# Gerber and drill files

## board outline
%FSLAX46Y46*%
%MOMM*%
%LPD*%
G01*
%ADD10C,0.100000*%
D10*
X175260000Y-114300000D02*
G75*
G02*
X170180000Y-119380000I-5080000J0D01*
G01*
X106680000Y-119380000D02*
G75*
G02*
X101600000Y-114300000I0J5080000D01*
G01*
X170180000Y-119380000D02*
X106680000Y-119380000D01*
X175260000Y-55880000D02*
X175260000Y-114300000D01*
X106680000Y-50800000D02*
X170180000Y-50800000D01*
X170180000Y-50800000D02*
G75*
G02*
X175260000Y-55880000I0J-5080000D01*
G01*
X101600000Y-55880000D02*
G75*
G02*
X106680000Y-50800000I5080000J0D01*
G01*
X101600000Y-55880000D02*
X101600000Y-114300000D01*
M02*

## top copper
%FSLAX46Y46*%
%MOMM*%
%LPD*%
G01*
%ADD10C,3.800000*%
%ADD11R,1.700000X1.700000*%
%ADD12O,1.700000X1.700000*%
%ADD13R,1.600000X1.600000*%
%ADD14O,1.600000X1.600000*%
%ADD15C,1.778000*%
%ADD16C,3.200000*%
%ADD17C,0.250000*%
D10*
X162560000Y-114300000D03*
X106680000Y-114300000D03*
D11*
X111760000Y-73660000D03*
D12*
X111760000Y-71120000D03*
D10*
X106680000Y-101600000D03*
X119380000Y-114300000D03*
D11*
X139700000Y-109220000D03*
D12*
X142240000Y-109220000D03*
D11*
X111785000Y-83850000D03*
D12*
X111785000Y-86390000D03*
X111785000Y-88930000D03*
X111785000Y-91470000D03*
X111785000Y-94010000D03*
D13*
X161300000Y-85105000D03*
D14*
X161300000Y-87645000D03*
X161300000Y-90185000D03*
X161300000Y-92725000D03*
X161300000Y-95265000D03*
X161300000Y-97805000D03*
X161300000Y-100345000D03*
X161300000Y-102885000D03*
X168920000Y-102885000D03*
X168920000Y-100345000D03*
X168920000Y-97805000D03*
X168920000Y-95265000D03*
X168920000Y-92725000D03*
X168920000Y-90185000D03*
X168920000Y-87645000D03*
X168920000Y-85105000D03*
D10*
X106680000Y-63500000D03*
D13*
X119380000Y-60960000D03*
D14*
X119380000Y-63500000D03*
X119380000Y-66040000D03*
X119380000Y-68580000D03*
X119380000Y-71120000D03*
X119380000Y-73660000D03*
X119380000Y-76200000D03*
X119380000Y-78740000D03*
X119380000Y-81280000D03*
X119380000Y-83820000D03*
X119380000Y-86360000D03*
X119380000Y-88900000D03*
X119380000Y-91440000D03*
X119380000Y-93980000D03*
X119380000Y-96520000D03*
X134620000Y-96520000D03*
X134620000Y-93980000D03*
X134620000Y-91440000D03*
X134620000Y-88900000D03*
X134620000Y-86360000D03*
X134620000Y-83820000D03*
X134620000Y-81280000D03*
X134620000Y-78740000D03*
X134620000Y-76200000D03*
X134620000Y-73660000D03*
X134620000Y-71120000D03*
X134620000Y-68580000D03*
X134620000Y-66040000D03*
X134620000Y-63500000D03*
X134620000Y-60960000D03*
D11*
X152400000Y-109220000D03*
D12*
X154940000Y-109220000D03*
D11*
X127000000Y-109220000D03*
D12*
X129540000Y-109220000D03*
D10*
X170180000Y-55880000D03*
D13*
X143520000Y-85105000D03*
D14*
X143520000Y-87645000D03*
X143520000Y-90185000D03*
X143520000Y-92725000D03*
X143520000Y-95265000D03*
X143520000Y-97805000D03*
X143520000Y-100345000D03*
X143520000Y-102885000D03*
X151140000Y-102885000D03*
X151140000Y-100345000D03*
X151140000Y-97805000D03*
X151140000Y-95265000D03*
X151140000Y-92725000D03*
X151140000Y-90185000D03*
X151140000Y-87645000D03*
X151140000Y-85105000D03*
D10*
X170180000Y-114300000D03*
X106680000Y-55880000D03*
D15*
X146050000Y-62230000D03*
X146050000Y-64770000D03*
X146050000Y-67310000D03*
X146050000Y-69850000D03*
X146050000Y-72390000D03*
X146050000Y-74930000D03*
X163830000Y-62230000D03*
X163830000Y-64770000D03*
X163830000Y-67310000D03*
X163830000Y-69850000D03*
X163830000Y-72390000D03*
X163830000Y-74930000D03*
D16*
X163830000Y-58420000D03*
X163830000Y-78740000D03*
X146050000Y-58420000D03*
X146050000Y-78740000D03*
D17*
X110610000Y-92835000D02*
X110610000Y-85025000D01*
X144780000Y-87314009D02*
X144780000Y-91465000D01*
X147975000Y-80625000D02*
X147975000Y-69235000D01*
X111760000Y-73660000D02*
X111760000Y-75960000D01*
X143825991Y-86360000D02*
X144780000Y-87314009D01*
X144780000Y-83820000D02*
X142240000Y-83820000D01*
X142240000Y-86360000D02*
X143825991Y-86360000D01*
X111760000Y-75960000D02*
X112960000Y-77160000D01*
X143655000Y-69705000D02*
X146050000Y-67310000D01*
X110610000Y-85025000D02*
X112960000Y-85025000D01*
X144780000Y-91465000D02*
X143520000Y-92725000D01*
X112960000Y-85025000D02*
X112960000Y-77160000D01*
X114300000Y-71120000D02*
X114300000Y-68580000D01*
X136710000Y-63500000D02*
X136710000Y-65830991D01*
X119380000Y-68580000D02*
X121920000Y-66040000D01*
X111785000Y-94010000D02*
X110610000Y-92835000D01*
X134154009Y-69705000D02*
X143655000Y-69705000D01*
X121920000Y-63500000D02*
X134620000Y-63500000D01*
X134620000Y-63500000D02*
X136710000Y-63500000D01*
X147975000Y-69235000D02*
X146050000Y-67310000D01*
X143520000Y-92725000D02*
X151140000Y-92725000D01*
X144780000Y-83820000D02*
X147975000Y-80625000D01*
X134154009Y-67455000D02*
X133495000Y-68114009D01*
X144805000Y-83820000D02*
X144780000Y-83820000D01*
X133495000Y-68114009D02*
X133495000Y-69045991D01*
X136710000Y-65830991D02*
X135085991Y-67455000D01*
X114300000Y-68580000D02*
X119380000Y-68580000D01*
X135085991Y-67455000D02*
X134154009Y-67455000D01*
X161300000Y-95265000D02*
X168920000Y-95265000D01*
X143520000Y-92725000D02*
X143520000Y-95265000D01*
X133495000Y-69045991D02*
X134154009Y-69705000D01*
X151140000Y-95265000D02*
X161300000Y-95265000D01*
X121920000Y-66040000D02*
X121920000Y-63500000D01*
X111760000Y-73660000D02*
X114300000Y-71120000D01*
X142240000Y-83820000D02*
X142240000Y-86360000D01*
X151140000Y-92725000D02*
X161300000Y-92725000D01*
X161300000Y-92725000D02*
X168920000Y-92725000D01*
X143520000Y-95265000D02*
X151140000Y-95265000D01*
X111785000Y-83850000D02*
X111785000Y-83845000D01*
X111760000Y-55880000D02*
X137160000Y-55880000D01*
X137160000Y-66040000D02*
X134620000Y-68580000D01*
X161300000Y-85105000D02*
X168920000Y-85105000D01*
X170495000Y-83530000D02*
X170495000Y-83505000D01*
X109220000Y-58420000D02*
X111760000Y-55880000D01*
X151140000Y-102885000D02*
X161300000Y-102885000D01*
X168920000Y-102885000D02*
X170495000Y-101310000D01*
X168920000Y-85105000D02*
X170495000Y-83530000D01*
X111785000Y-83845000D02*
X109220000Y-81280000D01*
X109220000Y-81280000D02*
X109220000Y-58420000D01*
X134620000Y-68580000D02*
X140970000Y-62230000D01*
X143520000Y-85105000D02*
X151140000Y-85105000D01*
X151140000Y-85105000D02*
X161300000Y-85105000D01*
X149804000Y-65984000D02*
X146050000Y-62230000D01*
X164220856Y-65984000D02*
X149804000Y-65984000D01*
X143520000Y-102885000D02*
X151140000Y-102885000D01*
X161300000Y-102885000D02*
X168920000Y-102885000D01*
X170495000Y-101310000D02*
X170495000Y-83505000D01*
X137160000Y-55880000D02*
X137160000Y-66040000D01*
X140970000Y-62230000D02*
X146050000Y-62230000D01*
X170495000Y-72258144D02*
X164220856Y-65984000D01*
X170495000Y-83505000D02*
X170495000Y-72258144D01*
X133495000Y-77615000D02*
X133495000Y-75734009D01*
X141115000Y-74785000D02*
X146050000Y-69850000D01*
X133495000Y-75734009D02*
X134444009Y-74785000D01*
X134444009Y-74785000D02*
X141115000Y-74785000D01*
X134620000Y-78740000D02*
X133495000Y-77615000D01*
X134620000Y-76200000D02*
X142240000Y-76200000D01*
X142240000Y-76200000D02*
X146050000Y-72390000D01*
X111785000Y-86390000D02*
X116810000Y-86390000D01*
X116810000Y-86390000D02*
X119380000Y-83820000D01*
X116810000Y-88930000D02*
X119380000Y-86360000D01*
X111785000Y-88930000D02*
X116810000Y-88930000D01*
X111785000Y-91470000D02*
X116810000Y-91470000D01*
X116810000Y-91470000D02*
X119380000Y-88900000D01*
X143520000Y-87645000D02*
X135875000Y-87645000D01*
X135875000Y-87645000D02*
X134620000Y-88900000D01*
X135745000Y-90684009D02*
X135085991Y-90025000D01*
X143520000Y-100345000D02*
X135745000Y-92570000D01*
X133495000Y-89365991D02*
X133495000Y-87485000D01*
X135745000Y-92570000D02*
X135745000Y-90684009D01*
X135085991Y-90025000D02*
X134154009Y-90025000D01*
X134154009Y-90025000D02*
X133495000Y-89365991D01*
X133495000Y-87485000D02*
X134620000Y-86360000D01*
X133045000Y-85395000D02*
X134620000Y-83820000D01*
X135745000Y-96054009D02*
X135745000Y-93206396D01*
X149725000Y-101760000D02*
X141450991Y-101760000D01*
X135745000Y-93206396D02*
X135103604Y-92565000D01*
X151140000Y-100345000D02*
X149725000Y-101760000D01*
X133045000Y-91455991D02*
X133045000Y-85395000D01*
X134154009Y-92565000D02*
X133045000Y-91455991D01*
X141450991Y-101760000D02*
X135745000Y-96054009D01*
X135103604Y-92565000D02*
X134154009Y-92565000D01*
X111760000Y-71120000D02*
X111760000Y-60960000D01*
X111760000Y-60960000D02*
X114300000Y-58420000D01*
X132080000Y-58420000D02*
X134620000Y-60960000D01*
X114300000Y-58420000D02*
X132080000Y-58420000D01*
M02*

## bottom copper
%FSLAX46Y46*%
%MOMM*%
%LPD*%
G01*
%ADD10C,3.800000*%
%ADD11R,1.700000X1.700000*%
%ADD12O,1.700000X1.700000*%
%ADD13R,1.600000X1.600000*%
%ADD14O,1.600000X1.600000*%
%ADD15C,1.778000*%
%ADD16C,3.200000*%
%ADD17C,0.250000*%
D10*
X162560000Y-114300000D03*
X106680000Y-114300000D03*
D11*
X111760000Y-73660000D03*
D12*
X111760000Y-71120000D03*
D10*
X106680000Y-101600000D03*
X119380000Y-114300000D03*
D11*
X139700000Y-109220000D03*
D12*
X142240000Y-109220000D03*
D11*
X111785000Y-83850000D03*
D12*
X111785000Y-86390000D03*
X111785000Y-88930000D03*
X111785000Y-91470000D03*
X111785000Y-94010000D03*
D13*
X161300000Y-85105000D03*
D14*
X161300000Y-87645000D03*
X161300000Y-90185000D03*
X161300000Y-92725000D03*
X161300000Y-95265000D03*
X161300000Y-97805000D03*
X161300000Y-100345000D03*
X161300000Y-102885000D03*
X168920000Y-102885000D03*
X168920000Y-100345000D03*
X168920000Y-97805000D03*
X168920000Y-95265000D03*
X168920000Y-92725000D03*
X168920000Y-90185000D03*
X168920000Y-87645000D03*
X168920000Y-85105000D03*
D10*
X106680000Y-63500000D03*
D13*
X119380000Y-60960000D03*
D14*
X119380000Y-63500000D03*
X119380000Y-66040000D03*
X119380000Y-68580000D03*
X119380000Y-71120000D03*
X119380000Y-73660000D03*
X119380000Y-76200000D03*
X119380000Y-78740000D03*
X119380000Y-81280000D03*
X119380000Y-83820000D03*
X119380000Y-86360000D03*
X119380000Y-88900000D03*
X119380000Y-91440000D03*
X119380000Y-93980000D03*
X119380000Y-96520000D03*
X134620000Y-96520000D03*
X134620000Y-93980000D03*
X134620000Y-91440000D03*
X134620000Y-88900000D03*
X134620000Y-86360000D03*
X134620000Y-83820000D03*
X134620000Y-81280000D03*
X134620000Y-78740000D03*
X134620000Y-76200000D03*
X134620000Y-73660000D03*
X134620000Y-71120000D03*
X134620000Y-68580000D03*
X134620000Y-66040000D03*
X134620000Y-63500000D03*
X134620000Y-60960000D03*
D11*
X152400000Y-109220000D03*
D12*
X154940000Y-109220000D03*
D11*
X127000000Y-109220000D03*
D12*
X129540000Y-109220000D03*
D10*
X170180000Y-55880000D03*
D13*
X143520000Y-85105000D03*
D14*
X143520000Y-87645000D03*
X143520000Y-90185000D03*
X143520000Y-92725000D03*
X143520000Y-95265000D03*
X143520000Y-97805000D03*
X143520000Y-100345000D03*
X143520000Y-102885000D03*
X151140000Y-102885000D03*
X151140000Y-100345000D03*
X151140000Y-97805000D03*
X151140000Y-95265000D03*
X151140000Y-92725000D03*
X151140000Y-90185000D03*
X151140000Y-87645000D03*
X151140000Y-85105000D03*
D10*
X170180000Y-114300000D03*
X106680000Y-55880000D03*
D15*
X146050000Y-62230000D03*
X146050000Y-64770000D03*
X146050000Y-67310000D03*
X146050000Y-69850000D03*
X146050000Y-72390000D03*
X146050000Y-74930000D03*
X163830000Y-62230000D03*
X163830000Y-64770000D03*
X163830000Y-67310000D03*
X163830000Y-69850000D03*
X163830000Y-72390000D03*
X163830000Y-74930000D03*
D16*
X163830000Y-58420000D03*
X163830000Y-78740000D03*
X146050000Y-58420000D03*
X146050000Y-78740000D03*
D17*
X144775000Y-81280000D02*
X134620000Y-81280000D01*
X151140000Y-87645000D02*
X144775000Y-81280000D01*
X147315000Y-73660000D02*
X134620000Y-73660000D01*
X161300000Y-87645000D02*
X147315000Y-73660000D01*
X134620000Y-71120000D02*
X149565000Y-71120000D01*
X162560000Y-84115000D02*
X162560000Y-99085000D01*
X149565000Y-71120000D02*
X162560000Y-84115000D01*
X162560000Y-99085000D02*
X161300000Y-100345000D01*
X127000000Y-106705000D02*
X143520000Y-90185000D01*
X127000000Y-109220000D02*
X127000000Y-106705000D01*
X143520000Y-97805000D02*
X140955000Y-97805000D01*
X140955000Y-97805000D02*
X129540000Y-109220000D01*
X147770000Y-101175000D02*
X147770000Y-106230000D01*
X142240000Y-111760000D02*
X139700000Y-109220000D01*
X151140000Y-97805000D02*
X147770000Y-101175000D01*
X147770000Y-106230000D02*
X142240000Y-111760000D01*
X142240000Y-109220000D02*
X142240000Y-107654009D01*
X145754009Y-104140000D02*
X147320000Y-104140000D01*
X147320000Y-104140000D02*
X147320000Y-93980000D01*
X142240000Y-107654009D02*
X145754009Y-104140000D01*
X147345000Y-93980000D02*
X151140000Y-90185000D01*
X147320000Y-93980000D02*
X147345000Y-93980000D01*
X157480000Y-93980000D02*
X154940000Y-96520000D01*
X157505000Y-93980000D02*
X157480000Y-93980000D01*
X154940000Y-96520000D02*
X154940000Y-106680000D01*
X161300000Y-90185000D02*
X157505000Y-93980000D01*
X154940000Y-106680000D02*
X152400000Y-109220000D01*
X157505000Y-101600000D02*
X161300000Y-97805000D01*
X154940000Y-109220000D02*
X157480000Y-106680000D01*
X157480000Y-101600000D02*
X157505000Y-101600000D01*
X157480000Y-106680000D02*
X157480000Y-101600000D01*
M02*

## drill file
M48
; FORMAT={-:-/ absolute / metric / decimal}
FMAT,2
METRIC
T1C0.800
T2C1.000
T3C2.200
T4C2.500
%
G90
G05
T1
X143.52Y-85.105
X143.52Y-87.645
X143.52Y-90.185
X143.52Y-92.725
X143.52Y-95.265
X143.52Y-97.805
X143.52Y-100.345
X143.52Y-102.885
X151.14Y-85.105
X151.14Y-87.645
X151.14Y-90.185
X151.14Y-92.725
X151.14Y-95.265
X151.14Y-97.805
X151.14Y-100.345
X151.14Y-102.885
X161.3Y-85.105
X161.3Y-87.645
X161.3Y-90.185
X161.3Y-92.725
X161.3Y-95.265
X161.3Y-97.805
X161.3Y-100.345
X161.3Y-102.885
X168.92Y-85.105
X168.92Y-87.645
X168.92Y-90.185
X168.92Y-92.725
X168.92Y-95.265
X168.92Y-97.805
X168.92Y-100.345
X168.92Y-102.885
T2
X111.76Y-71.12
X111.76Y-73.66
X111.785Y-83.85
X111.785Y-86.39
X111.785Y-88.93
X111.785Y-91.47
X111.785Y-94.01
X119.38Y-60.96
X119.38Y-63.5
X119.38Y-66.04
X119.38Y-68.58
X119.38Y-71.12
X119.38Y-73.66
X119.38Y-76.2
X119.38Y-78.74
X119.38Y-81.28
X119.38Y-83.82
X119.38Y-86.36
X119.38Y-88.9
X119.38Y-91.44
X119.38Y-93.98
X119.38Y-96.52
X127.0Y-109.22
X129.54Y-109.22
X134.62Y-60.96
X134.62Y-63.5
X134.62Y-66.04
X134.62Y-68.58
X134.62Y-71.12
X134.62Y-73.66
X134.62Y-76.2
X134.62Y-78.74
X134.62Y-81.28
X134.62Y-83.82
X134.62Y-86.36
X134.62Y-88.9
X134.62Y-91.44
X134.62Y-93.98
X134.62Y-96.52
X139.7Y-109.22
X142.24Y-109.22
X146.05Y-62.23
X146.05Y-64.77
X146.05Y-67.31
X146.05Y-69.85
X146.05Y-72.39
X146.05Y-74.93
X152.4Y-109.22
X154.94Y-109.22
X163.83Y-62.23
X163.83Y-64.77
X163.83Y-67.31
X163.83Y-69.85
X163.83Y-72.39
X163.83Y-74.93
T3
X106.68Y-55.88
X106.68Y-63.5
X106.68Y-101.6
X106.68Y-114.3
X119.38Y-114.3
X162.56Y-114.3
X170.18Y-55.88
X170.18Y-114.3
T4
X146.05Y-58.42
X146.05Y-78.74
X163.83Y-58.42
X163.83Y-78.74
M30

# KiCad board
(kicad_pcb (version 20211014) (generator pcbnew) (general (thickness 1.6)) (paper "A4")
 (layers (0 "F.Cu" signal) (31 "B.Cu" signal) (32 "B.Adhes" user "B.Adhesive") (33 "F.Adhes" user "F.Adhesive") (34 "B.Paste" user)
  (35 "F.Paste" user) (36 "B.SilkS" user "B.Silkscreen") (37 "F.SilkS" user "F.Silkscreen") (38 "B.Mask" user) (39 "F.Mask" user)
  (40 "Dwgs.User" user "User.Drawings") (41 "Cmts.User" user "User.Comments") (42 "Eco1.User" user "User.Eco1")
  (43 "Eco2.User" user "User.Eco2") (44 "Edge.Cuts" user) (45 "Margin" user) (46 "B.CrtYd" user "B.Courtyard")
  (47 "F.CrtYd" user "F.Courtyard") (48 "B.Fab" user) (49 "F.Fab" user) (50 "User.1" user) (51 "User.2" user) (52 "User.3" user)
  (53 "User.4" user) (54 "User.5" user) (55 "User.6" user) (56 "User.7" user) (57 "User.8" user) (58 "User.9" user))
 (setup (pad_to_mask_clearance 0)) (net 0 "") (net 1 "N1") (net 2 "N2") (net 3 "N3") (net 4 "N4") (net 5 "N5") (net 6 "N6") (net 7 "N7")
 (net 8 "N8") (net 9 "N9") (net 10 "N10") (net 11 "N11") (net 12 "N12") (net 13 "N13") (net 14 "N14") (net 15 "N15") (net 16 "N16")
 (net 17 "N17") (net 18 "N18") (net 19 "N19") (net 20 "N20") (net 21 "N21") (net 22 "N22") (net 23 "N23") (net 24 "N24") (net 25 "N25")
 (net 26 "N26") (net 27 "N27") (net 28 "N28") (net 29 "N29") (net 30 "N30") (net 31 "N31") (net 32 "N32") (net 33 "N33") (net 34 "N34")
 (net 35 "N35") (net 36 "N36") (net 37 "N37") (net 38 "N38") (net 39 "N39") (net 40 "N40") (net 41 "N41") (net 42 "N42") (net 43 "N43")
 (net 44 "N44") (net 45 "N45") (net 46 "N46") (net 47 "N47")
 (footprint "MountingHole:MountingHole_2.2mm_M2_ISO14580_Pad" (layer "F.Cu") (at 162.56 114.3)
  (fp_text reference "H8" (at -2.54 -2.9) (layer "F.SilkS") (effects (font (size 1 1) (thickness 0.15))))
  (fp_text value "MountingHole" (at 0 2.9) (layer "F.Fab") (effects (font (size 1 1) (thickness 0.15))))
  (pad "1" thru_hole circle (at 0 0) (size 3.8 3.8) (drill 2.2) (layers *.Cu *.Mask)))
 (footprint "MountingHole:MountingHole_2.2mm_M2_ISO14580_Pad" (layer "F.Cu") (at 106.68 114.3)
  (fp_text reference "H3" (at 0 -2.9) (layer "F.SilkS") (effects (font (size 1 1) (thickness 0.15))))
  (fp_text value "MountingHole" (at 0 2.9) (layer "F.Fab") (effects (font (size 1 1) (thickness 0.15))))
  (pad "1" thru_hole circle (at 0 0) (size 3.8 3.8) (drill 2.2) (layers *.Cu *.Mask)))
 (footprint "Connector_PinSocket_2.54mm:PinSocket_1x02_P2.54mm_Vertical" (layer "F.Cu") (at 111.76 73.66 180)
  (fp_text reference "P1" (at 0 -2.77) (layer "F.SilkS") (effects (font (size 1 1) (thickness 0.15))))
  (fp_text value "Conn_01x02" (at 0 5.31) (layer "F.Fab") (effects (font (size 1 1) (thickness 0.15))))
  (pad "1" thru_hole rect (at 0 0 180) (size 1.7 1.7) (drill 1) (layers *.Cu *.Mask) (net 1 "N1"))
  (pad "2" thru_hole oval (at 0 2.54 180) (size 1.7 1.7) (drill 1) (layers *.Cu *.Mask) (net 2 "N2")))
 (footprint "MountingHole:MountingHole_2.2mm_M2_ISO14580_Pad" (layer "F.Cu") (at 106.68 101.6)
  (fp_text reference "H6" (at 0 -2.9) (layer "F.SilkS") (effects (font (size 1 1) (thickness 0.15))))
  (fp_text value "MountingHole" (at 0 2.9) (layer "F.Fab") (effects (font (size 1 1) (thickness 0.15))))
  (pad "1" thru_hole circle (at 0 0) (size 3.8 3.8) (drill 2.2) (layers *.Cu *.Mask)))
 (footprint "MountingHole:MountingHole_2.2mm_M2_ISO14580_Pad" (layer "F.Cu") (at 119.38 114.3)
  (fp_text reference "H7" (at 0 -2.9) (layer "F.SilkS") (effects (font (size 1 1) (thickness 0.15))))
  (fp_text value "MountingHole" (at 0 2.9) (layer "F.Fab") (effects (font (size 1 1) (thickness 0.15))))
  (pad "1" thru_hole circle (at 0 0) (size 3.8 3.8) (drill 2.2) (layers *.Cu *.Mask)))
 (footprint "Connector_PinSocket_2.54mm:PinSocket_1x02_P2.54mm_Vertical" (layer "F.Cu") (at 139.7 109.22 90)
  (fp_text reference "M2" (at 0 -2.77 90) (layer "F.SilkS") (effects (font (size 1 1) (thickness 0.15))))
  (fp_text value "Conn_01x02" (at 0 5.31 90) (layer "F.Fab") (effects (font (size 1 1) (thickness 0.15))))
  (pad "1" thru_hole rect (at 0 0 90) (size 1.7 1.7) (drill 1) (layers *.Cu *.Mask) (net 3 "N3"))
  (pad "2" thru_hole oval (at 0 2.54 90) (size 1.7 1.7) (drill 1) (layers *.Cu *.Mask) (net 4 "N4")))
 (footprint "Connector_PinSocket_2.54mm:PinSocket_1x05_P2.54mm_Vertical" (layer "F.Cu") (at 111.785 83.85)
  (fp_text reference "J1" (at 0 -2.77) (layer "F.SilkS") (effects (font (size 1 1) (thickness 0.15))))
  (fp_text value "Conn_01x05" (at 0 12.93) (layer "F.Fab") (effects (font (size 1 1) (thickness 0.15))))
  (pad "1" thru_hole rect (at 0 0) (size 1.7 1.7) (drill 1) (layers *.Cu *.Mask) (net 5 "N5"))
  (pad "2" thru_hole oval (at 0 2.54) (size 1.7 1.7) (drill 1) (layers *.Cu *.Mask) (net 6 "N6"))
  (pad "3" thru_hole oval (at 0 5.08) (size 1.7 1.7) (drill 1) (layers *.Cu *.Mask) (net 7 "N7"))
  (pad "4" thru_hole oval (at 0 7.62) (size 1.7 1.7) (drill 1) (layers *.Cu *.Mask) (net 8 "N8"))
  (pad "5" thru_hole oval (at 0 10.16) (size 1.7 1.7) (drill 1) (layers *.Cu *.Mask) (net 1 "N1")))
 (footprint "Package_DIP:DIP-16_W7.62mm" (layer "F.Cu") (at 161.3 85.105)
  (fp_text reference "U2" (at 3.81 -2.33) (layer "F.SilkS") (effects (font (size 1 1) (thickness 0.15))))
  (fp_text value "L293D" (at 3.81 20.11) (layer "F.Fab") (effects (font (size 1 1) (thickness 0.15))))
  (pad "1" thru_hole rect (at 0 0) (size 1.6 1.6) (drill 0.8) (layers *.Cu *.Mask) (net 5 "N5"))
  (pad "2" thru_hole oval (at 0 2.54) (size 1.6 1.6) (drill 0.8) (layers *.Cu *.Mask) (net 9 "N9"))
  (pad "3" thru_hole oval (at 0 5.08) (size 1.6 1.6) (drill 0.8) (layers *.Cu *.Mask) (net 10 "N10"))
  (pad "4" thru_hole oval (at 0 7.62) (size 1.6 1.6) (drill 0.8) (layers *.Cu *.Mask) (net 1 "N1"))
  (pad "5" thru_hole oval (at 0 10.16) (size 1.6 1.6) (drill 0.8) (layers *.Cu *.Mask) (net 1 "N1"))
  (pad "6" thru_hole oval (at 0 12.7) (size 1.6 1.6) (drill 0.8) (layers *.Cu *.Mask) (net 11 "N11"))
  (pad "7" thru_hole oval (at 0 15.24) (size 1.6 1.6) (drill 0.8) (layers *.Cu *.Mask) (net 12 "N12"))
  (pad "8" thru_hole oval (at 0 17.78) (size 1.6 1.6) (drill 0.8) (layers *.Cu *.Mask) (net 5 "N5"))
  (pad "9" thru_hole oval (at 7.62 17.78) (size 1.6 1.6) (drill 0.8) (layers *.Cu *.Mask) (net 5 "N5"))
  (pad "10" thru_hole oval (at 7.62 15.24) (size 1.6 1.6) (drill 0.8) (layers *.Cu *.Mask) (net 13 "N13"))
  (pad "11" thru_hole oval (at 7.62 12.7) (size 1.6 1.6) (drill 0.8) (layers *.Cu *.Mask) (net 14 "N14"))
  (pad "12" thru_hole oval (at 7.62 10.16) (size 1.6 1.6) (drill 0.8) (layers *.Cu *.Mask) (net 1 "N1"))
  (pad "13" thru_hole oval (at 7.62 7.62) (size 1.6 1.6) (drill 0.8) (layers *.Cu *.Mask) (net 1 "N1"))
  (pad "14" thru_hole oval (at 7.62 5.08) (size 1.6 1.6) (drill 0.8) (layers *.Cu *.Mask) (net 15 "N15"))
  (pad "15" thru_hole oval (at 7.62 2.54) (size 1.6 1.6) (drill 0.8) (layers *.Cu *.Mask) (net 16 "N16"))
  (pad "16" thru_hole oval (at 7.62 0) (size 1.6 1.6) (drill 0.8) (layers *.Cu *.Mask) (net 5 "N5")))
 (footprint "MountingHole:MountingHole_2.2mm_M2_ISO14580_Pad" (layer "F.Cu") (at 106.68 63.5)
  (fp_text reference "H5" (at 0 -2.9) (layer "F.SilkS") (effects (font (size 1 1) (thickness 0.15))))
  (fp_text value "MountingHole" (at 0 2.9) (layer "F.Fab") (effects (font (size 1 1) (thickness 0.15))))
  (pad "1" thru_hole circle (at 0 0) (size 3.8 3.8) (drill 2.2) (layers *.Cu *.Mask)))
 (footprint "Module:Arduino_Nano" (layer "F.Cu") (at 119.38 60.96)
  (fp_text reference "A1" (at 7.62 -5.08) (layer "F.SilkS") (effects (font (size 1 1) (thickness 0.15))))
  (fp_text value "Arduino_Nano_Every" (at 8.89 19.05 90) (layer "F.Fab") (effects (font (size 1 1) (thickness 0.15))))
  (pad "1" thru_hole rect (at 0 0) (size 1.6 1.6) (drill 1) (layers *.Cu *.Mask) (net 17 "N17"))
  (pad "2" thru_hole oval (at 0 2.54) (size 1.6 1.6) (drill 1) (layers *.Cu *.Mask) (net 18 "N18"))
  (pad "3" thru_hole oval (at 0 5.08) (size 1.6 1.6) (drill 1) (layers *.Cu *.Mask) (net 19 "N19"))
  (pad "4" thru_hole oval (at 0 7.62) (size 1.6 1.6) (drill 1) (layers *.Cu *.Mask) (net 1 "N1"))
  (pad "5" thru_hole oval (at 0 10.16) (size 1.6 1.6) (drill 1) (layers *.Cu *.Mask) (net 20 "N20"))
  (pad "6" thru_hole oval (at 0 12.7) (size 1.6 1.6) (drill 1) (layers *.Cu *.Mask) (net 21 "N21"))
  (pad "7" thru_hole oval (at 0 15.24) (size 1.6 1.6) (drill 1) (layers *.Cu *.Mask) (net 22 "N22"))
  (pad "8" thru_hole oval (at 0 17.78) (size 1.6 1.6) (drill 1) (layers *.Cu *.Mask) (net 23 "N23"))
  (pad "9" thru_hole oval (at 0 20.32) (size 1.6 1.6) (drill 1) (layers *.Cu *.Mask) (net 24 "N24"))
  (pad "10" thru_hole oval (at 0 22.86) (size 1.6 1.6) (drill 1) (layers *.Cu *.Mask) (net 6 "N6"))
  (pad "11" thru_hole oval (at 0 25.4) (size 1.6 1.6) (drill 1) (layers *.Cu *.Mask) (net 7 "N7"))
  (pad "12" thru_hole oval (at 0 27.94) (size 1.6 1.6) (drill 1) (layers *.Cu *.Mask) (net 8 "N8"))
  (pad "13" thru_hole oval (at 0 30.48) (size 1.6 1.6) (drill 1) (layers *.Cu *.Mask) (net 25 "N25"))
  (pad "14" thru_hole oval (at 0 33.02) (size 1.6 1.6) (drill 1) (layers *.Cu *.Mask) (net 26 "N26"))
  (pad "15" thru_hole oval (at 0 35.56) (size 1.6 1.6) (drill 1) (layers *.Cu *.Mask) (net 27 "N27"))
  (pad "16" thru_hole oval (at 15.24 35.56) (size 1.6 1.6) (drill 1) (layers *.Cu *.Mask) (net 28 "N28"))
  (pad "17" thru_hole oval (at 15.24 33.02) (size 1.6 1.6) (drill 1) (layers *.Cu *.Mask) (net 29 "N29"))
  (pad "18" thru_hole oval (at 15.24 30.48) (size 1.6 1.6) (drill 1) (layers *.Cu *.Mask) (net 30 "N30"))
  (pad "19" thru_hole oval (at 15.24 27.94) (size 1.6 1.6) (drill 1) (layers *.Cu *.Mask) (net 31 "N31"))
  (pad "20" thru_hole oval (at 15.24 25.4) (size 1.6 1.6) (drill 1) (layers *.Cu *.Mask) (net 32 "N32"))
  (pad "21" thru_hole oval (at 15.24 22.86) (size 1.6 1.6) (drill 1) (layers *.Cu *.Mask) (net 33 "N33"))
  (pad "22" thru_hole oval (at 15.24 20.32) (size 1.6 1.6) (drill 1) (layers *.Cu *.Mask) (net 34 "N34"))
  (pad "23" thru_hole oval (at 15.24 17.78) (size 1.6 1.6) (drill 1) (layers *.Cu *.Mask) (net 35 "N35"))
  (pad "24" thru_hole oval (at 15.24 15.24) (size 1.6 1.6) (drill 1) (layers *.Cu *.Mask) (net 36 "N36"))
  (pad "25" thru_hole oval (at 15.24 12.7) (size 1.6 1.6) (drill 1) (layers *.Cu *.Mask) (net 9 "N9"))
  (pad "26" thru_hole oval (at 15.24 10.16) (size 1.6 1.6) (drill 1) (layers *.Cu *.Mask) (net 12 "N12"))
  (pad "27" thru_hole oval (at 15.24 7.62) (size 1.6 1.6) (drill 1) (layers *.Cu *.Mask) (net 5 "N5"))
  (pad "28" thru_hole oval (at 15.24 5.08) (size 1.6 1.6) (drill 1) (layers *.Cu *.Mask) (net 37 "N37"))
  (pad "29" thru_hole oval (at 15.24 2.54) (size 1.6 1.6) (drill 1) (layers *.Cu *.Mask) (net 1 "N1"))
  (pad "30" thru_hole oval (at 15.24 0) (size 1.6 1.6) (drill 1) (layers *.Cu *.Mask) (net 2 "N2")))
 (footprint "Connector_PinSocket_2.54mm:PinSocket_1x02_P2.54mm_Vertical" (layer "F.Cu") (at 152.4 109.22 90)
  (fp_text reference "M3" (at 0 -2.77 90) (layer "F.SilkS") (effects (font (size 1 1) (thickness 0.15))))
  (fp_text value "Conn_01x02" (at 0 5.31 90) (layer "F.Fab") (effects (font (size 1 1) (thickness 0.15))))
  (pad "1" thru_hole rect (at 0 0 90) (size 1.7 1.7) (drill 1) (layers *.Cu *.Mask) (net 10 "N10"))
  (pad "2" thru_hole oval (at 0 2.54 90) (size 1.7 1.7) (drill 1) (layers *.Cu *.Mask) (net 11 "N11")))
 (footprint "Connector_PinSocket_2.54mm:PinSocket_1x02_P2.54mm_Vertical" (layer "F.Cu") (at 127 109.22 90)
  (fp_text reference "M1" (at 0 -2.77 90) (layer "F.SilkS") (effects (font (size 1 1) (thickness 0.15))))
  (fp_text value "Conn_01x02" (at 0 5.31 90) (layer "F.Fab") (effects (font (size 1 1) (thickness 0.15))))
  (pad "1" thru_hole rect (at 0 0 90) (size 1.7 1.7) (drill 1) (layers *.Cu *.Mask) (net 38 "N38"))
  (pad "2" thru_hole oval (at 0 2.54 90) (size 1.7 1.7) (drill 1) (layers *.Cu *.Mask) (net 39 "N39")))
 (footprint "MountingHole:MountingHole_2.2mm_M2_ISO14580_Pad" (layer "F.Cu") (at 170.18 55.88)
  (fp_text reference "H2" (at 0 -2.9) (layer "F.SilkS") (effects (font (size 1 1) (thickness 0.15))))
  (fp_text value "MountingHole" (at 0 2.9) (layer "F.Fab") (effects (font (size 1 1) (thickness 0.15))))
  (pad "1" thru_hole circle (at 0 0) (size 3.8 3.8) (drill 2.2) (layers *.Cu *.Mask)))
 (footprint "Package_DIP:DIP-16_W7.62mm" (layer "F.Cu") (at 143.52 85.105)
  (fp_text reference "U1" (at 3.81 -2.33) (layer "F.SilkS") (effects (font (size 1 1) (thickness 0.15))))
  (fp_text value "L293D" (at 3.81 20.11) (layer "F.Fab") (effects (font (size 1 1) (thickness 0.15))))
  (pad "1" thru_hole rect (at 0 0) (size 1.6 1.6) (drill 0.8) (layers *.Cu *.Mask) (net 5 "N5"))
  (pad "2" thru_hole oval (at 0 2.54) (size 1.6 1.6) (drill 0.8) (layers *.Cu *.Mask) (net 31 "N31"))
  (pad "3" thru_hole oval (at 0 5.08) (size 1.6 1.6) (drill 0.8) (layers *.Cu *.Mask) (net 38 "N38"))
  (pad "4" thru_hole oval (at 0 7.62) (size 1.6 1.6) (drill 0.8) (layers *.Cu *.Mask) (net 1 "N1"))
  (pad "5" thru_hole oval (at 0 10.16) (size 1.6 1.6) (drill 0.8) (layers *.Cu *.Mask) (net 1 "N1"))
  (pad "6" thru_hole oval (at 0 12.7) (size 1.6 1.6) (drill 0.8) (layers *.Cu *.Mask) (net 39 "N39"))
  (pad "7" thru_hole oval (at 0 15.24) (size 1.6 1.6) (drill 0.8) (layers *.Cu *.Mask) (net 32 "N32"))
  (pad "8" thru_hole oval (at 0 17.78) (size 1.6 1.6) (drill 0.8) (layers *.Cu *.Mask) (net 5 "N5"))
  (pad "9" thru_hole oval (at 7.62 17.78) (size 1.6 1.6) (drill 0.8) (layers *.Cu *.Mask) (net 5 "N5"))
  (pad "10" thru_hole oval (at 7.62 15.24) (size 1.6 1.6) (drill 0.8) (layers *.Cu *.Mask) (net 33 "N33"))
  (pad "11" thru_hole oval (at 7.62 12.7) (size 1.6 1.6) (drill 0.8) (layers *.Cu *.Mask) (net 3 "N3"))
  (pad "12" thru_hole oval (at 7.62 10.16) (size 1.6 1.6) (drill 0.8) (layers *.Cu *.Mask) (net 1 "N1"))
  (pad "13" thru_hole oval (at 7.62 7.62) (size 1.6 1.6) (drill 0.8) (layers *.Cu *.Mask) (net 1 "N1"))
  (pad "14" thru_hole oval (at 7.62 5.08) (size 1.6 1.6) (drill 0.8) (layers *.Cu *.Mask) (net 4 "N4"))
  (pad "15" thru_hole oval (at 7.62 2.54) (size 1.6 1.6) (drill 0.8) (layers *.Cu *.Mask) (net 34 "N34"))
  (pad "16" thru_hole oval (at 7.62 0) (size 1.6 1.6) (drill 0.8) (layers *.Cu *.Mask) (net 5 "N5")))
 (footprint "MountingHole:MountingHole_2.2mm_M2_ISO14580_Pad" (layer "F.Cu") (at 170.18 114.3)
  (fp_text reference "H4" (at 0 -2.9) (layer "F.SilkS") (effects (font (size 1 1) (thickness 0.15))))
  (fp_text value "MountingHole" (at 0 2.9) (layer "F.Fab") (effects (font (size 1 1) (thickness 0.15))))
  (pad "1" thru_hole circle (at 0 0) (size 3.8 3.8) (drill 2.2) (layers *.Cu *.Mask)))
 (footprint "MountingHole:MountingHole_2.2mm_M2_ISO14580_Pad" (layer "F.Cu") (at 106.68 55.88)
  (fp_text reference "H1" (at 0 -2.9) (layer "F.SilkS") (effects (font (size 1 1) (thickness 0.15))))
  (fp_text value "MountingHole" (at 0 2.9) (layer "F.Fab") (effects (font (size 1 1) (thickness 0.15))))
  (pad "1" thru_hole circle (at 0 0) (size 3.8 3.8) (drill 2.2) (layers *.Cu *.Mask)))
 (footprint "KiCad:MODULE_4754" (layer "F.Cu") (at 154.94 68.58 -90)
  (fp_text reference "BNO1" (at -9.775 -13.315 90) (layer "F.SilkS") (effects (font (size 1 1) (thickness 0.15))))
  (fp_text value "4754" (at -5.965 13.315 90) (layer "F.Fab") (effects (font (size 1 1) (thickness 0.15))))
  (pad "JP1_1" thru_hole circle locked (at -6.35 8.89 270) (size 1.778 1.778) (drill 1) (layers *.Cu *.Mask) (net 5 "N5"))
  (pad "JP1_2" thru_hole circle locked (at -3.81 8.89 270) (size 1.778 1.778) (drill 1) (layers *.Cu *.Mask) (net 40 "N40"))
  (pad "JP1_3" thru_hole circle locked (at -1.27 8.89 270) (size 1.778 1.778) (drill 1) (layers *.Cu *.Mask) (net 1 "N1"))
  (pad "JP1_4" thru_hole circle locked (at 1.27 8.89 270) (size 1.778 1.778) (drill 1) (layers *.Cu *.Mask) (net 35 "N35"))
  (pad "JP1_5" thru_hole circle locked (at 3.81 8.89 270) (size 1.778 1.778) (drill 1) (layers *.Cu *.Mask) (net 36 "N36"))
  (pad "JP1_6" thru_hole circle locked (at 6.35 8.89 270) (size 1.778 1.778) (drill 1) (layers *.Cu *.Mask) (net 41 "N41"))
  (pad "JP2_1" thru_hole circle locked (at -6.35 -8.89 270) (size 1.778 1.778) (drill 1) (layers *.Cu *.Mask) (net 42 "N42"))
  (pad "JP2_2" thru_hole circle locked (at -3.81 -8.89 270) (size 1.778 1.778) (drill 1) (layers *.Cu *.Mask) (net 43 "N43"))
  (pad "JP2_3" thru_hole circle locked (at -1.27 -8.89 270) (size 1.778 1.778) (drill 1) (layers *.Cu *.Mask) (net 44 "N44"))
  (pad "JP2_4" thru_hole circle locked (at 1.27 -8.89 270) (size 1.778 1.778) (drill 1) (layers *.Cu *.Mask) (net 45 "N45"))
  (pad "JP2_5" thru_hole circle locked (at 3.81 -8.89 270) (size 1.778 1.778) (drill 1) (layers *.Cu *.Mask) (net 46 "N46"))
  (pad "JP2_6" thru_hole circle locked (at 6.35 -8.89 270) (size 1.778 1.778) (drill 1) (layers *.Cu *.Mask) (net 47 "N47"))
  (pad "P1" thru_hole circle locked (at -10.16 -8.89 270) (size 3.2 3.2) (drill 2.5) (layers *.Cu *.Mask))
  (pad "P2" thru_hole circle locked (at 10.16 -8.89 270) (size 3.2 3.2) (drill 2.5) (layers *.Cu *.Mask))
  (pad "P3" thru_hole circle locked (at -10.16 8.89 270) (size 3.2 3.2) (drill 2.5) (layers *.Cu *.Mask))
  (pad "P4" thru_hole circle locked (at 10.16 8.89 270) (size 3.2 3.2) (drill 2.5) (layers *.Cu *.Mask)))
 (gr_arc (start 175.26 114.3) (mid 173.772102 117.892102) (end 170.18 119.38) (layer "Edge.Cuts") (width 0.1))
 (gr_arc (start 106.68 119.38) (mid 103.087898 117.892102) (end 101.6 114.3) (layer "Edge.Cuts") (width 0.1))
 (gr_line (start 170.18 119.38) (end 106.68 119.38) (layer "Edge.Cuts") (width 0.1))
 (gr_line (start 175.26 55.88) (end 175.26 114.3) (layer "Edge.Cuts") (width 0.1))
 (gr_line (start 106.68 50.8) (end 170.18 50.8) (layer "Edge.Cuts") (width 0.1))
 (gr_arc (start 170.18 50.8) (mid 173.772102 52.287898) (end 175.26 55.88) (layer "Edge.Cuts") (width 0.1))
 (gr_arc (start 101.6 55.88) (mid 103.087898 52.287898) (end 106.68 50.8) (layer "Edge.Cuts") (width 0.1))
 (gr_line (start 101.6 55.88) (end 101.6 114.3) (layer "Edge.Cuts") (width 0.1))
 (segment (start 110.61 92.835) (end 110.61 85.025) (width 0.25) (layer "F.Cu") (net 1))
 (segment (start 144.78 87.314009) (end 144.78 91.465) (width 0.25) (layer "F.Cu") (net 1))
 (segment (start 147.975 80.625) (end 147.975 69.235) (width 0.25) (layer "F.Cu") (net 1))
 (segment (start 111.76 73.66) (end 111.76 75.96) (width 0.25) (layer "F.Cu") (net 1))
 (segment (start 143.825991 86.36) (end 144.78 87.314009) (width 0.25) (layer "F.Cu") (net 1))
 (segment (start 144.78 83.82) (end 142.24 83.82) (width 0.25) (layer "F.Cu") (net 1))
 (segment (start 142.24 86.36) (end 143.825991 86.36) (width 0.25) (layer "F.Cu") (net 1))
 (segment (start 111.76 75.96) (end 112.96 77.16) (width 0.25) (layer "F.Cu") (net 1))
 (segment (start 143.655 69.705) (end 146.05 67.31) (width 0.25) (layer "F.Cu") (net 1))
 (segment (start 110.61 85.025) (end 112.96 85.025) (width 0.25) (layer "F.Cu") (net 1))
 (segment (start 144.78 91.465) (end 143.52 92.725) (width 0.25) (layer "F.Cu") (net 1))
 (segment (start 112.96 85.025) (end 112.96 77.16) (width 0.25) (layer "F.Cu") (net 1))
 (segment (start 114.3 71.12) (end 114.3 68.58) (width 0.25) (layer "F.Cu") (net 1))
 (segment (start 136.71 63.5) (end 136.71 65.830991) (width 0.25) (layer "F.Cu") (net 1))
 (segment (start 119.38 68.58) (end 121.92 66.04) (width 0.25) (layer "F.Cu") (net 1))
 (segment (start 111.785 94.01) (end 110.61 92.835) (width 0.25) (layer "F.Cu") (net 1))
 (segment (start 134.154009 69.705) (end 143.655 69.705) (width 0.25) (layer "F.Cu") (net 1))
 (segment (start 121.92 63.5) (end 134.62 63.5) (width 0.25) (layer "F.Cu") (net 1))
 (segment (start 134.62 63.5) (end 136.71 63.5) (width 0.25) (layer "F.Cu") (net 1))
 (segment (start 147.975 69.235) (end 146.05 67.31) (width 0.25) (layer "F.Cu") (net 1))
 (segment (start 143.52 92.725) (end 151.14 92.725) (width 0.25) (layer "F.Cu") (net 1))
 (segment (start 144.78 83.82) (end 147.975 80.625) (width 0.25) (layer "F.Cu") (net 1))
 (segment (start 134.154009 67.455) (end 133.495 68.114009) (width 0.25) (layer "F.Cu") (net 1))
 (segment (start 144.805 83.82) (end 144.78 83.82) (width 0.25) (layer "F.Cu") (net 1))
 (segment (start 133.495 68.114009) (end 133.495 69.045991) (width 0.25) (layer "F.Cu") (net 1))
 (segment (start 136.71 65.830991) (end 135.085991 67.455) (width 0.25) (layer "F.Cu") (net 1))
 (segment (start 114.3 68.58) (end 119.38 68.58) (width 0.25) (layer "F.Cu") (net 1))
 (segment (start 135.085991 67.455) (end 134.154009 67.455) (width 0.25) (layer "F.Cu") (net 1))
 (segment (start 161.3 95.265) (end 168.92 95.265) (width 0.25) (layer "F.Cu") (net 1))
 (segment (start 143.52 92.725) (end 143.52 95.265) (width 0.25) (layer "F.Cu") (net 1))
 (segment (start 133.495 69.045991) (end 134.154009 69.705) (width 0.25) (layer "F.Cu") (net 1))
 (segment (start 151.14 95.265) (end 161.3 95.265) (width 0.25) (layer "F.Cu") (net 1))
 (segment (start 121.92 66.04) (end 121.92 63.5) (width 0.25) (layer "F.Cu") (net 1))
 (segment (start 111.76 73.66) (end 114.3 71.12) (width 0.25) (layer "F.Cu") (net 1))
 (segment (start 142.24 83.82) (end 142.24 86.36) (width 0.25) (layer "F.Cu") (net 1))
 (segment (start 151.14 92.725) (end 161.3 92.725) (width 0.25) (layer "F.Cu") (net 1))
 (segment (start 161.3 92.725) (end 168.92 92.725) (width 0.25) (layer "F.Cu") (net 1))
 (segment (start 143.52 95.265) (end 151.14 95.265) (width 0.25) (layer "F.Cu") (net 1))
 (segment (start 111.785 83.85) (end 111.785 83.845) (width 0.25) (layer "F.Cu") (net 5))
 (segment (start 111.76 55.88) (end 137.16 55.88) (width 0.25) (layer "F.Cu") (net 5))
 (segment (start 137.16 66.04) (end 134.62 68.58) (width 0.25) (layer "F.Cu") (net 5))
 (segment (start 161.3 85.105) (end 168.92 85.105) (width 0.25) (layer "F.Cu") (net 5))
 (segment (start 170.495 83.53) (end 170.495 83.505) (width 0.25) (layer "F.Cu") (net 5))
 (segment (start 109.22 58.42) (end 111.76 55.88) (width 0.25) (layer "F.Cu") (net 5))
 (segment (start 151.14 102.885) (end 161.3 102.885) (width 0.25) (layer "F.Cu") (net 5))
 (segment (start 168.92 102.885) (end 170.495 101.31) (width 0.25) (layer "F.Cu") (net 5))
 (segment (start 168.92 85.105) (end 170.495 83.53) (width 0.25) (layer "F.Cu") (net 5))
 (segment (start 111.785 83.845) (end 109.22 81.28) (width 0.25) (layer "F.Cu") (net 5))
 (segment (start 109.22 81.28) (end 109.22 58.42) (width 0.25) (layer "F.Cu") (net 5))
 (segment (start 134.62 68.58) (end 140.97 62.23) (width 0.25) (layer "F.Cu") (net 5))
 (segment (start 143.52 85.105) (end 151.14 85.105) (width 0.25) (layer "F.Cu") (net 5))
 (segment (start 151.14 85.105) (end 161.3 85.105) (width 0.25) (layer "F.Cu") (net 5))
 (segment (start 149.804 65.984) (end 146.05 62.23) (width 0.25) (layer "F.Cu") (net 5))
 (segment (start 164.220856 65.984) (end 149.804 65.984) (width 0.25) (layer "F.Cu") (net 5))
 (segment (start 143.52 102.885) (end 151.14 102.885) (width 0.25) (layer "F.Cu") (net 5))
 (segment (start 161.3 102.885) (end 168.92 102.885) (width 0.25) (layer "F.Cu") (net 5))
 (segment (start 170.495 101.31) (end 170.495 83.505) (width 0.25) (layer "F.Cu") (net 5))
 (segment (start 137.16 55.88) (end 137.16 66.04) (width 0.25) (layer "F.Cu") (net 5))
 (segment (start 140.97 62.23) (end 146.05 62.23) (width 0.25) (layer "F.Cu") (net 5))
 (segment (start 170.495 72.258144) (end 164.220856 65.984) (width 0.25) (layer "F.Cu") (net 5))
 (segment (start 170.495 83.505) (end 170.495 72.258144) (width 0.25) (layer "F.Cu") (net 5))
 (segment (start 133.495 77.615) (end 133.495 75.734009) (width 0.25) (layer "F.Cu") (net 35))
 (segment (start 141.115 74.785) (end 146.05 69.85) (width 0.25) (layer "F.Cu") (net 35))
 (segment (start 133.495 75.734009) (end 134.444009 74.785) (width 0.25) (layer "F.Cu") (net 35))
 (segment (start 134.444009 74.785) (end 141.115 74.785) (width 0.25) (layer "F.Cu") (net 35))
 (segment (start 134.62 78.74) (end 133.495 77.615) (width 0.25) (layer "F.Cu") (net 35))
 (segment (start 134.62 76.2) (end 142.24 76.2) (width 0.25) (layer "F.Cu") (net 36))
 (segment (start 142.24 76.2) (end 146.05 72.39) (width 0.25) (layer "F.Cu") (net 36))
 (segment (start 111.785 86.39) (end 116.81 86.39) (width 0.25) (layer "F.Cu") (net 6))
 (segment (start 116.81 86.39) (end 119.38 83.82) (width 0.25) (layer "F.Cu") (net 6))
 (segment (start 116.81 88.93) (end 119.38 86.36) (width 0.25) (layer "F.Cu") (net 7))
 (segment (start 111.785 88.93) (end 116.81 88.93) (width 0.25) (layer "F.Cu") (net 7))
 (segment (start 111.785 91.47) (end 116.81 91.47) (width 0.25) (layer "F.Cu") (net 8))
 (segment (start 116.81 91.47) (end 119.38 88.9) (width 0.25) (layer "F.Cu") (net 8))
 (segment (start 143.52 87.645) (end 135.875 87.645) (width 0.25) (layer "F.Cu") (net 31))
 (segment (start 135.875 87.645) (end 134.62 88.9) (width 0.25) (layer "F.Cu") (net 31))
 (segment (start 135.745 90.684009) (end 135.085991 90.025) (width 0.25) (layer "F.Cu") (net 32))
 (segment (start 143.52 100.345) (end 135.745 92.57) (width 0.25) (layer "F.Cu") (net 32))
 (segment (start 133.495 89.365991) (end 133.495 87.485) (width 0.25) (layer "F.Cu") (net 32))
 (segment (start 135.745 92.57) (end 135.745 90.684009) (width 0.25) (layer "F.Cu") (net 32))
 (segment (start 135.085991 90.025) (end 134.154009 90.025) (width 0.25) (layer "F.Cu") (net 32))
 (segment (start 134.154009 90.025) (end 133.495 89.365991) (width 0.25) (layer "F.Cu") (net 32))
 (segment (start 133.495 87.485) (end 134.62 86.36) (width 0.25) (layer "F.Cu") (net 32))
 (segment (start 133.045 85.395) (end 134.62 83.82) (width 0.25) (layer "F.Cu") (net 33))
 (segment (start 135.745 96.054009) (end 135.745 93.206396) (width 0.25) (layer "F.Cu") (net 33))
 (segment (start 149.725 101.76) (end 141.450991 101.76) (width 0.25) (layer "F.Cu") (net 33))
 (segment (start 135.745 93.206396) (end 135.103604 92.565) (width 0.25) (layer "F.Cu") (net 33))
 (segment (start 151.14 100.345) (end 149.725 101.76) (width 0.25) (layer "F.Cu") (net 33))
 (segment (start 133.045 91.455991) (end 133.045 85.395) (width 0.25) (layer "F.Cu") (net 33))
 (segment (start 134.154009 92.565) (end 133.045 91.455991) (width 0.25) (layer "F.Cu") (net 33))
 (segment (start 141.450991 101.76) (end 135.745 96.054009) (width 0.25) (layer "F.Cu") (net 33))
 (segment (start 135.103604 92.565) (end 134.154009 92.565) (width 0.25) (layer "F.Cu") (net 33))
 (segment (start 144.775 81.28) (end 134.62 81.28) (width 0.25) (layer "B.Cu") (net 34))
 (segment (start 151.14 87.645) (end 144.775 81.28) (width 0.25) (layer "B.Cu") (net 34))
 (segment (start 147.315 73.66) (end 134.62 73.66) (width 0.25) (layer "B.Cu") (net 9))
 (segment (start 161.3 87.645) (end 147.315 73.66) (width 0.25) (layer "B.Cu") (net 9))
 (segment (start 134.62 71.12) (end 149.565 71.12) (width 0.25) (layer "B.Cu") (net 12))
 (segment (start 162.56 84.115) (end 162.56 99.085) (width 0.25) (layer "B.Cu") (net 12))
 (segment (start 149.565 71.12) (end 162.56 84.115) (width 0.25) (layer "B.Cu") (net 12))
 (segment (start 162.56 99.085) (end 161.3 100.345) (width 0.25) (layer "B.Cu") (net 12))
 (segment (start 111.76 71.12) (end 111.76 60.96) (width 0.25) (layer "F.Cu") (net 2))
 (segment (start 111.76 60.96) (end 114.3 58.42) (width 0.25) (layer "F.Cu") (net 2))
 (segment (start 132.08 58.42) (end 134.62 60.96) (width 0.25) (layer "F.Cu") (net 2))
 (segment (start 114.3 58.42) (end 132.08 58.42) (width 0.25) (layer "F.Cu") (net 2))
 (segment (start 127 106.705) (end 143.52 90.185) (width 0.25) (layer "B.Cu") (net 38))
 (segment (start 127 109.22) (end 127 106.705) (width 0.25) (layer "B.Cu") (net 38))
 (segment (start 143.52 97.805) (end 140.955 97.805) (width 0.25) (layer "B.Cu") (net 39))
 (segment (start 140.955 97.805) (end 129.54 109.22) (width 0.25) (layer "B.Cu") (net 39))
 (segment (start 147.77 101.175) (end 147.77 106.23) (width 0.25) (layer "B.Cu") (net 3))
 (segment (start 142.24 111.76) (end 139.7 109.22) (width 0.25) (layer "B.Cu") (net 3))
 (segment (start 151.14 97.805) (end 147.77 101.175) (width 0.25) (layer "B.Cu") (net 3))
 (segment (start 147.77 106.23) (end 142.24 111.76) (width 0.25) (layer "B.Cu") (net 3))
 (segment (start 142.24 109.22) (end 142.24 107.654009) (width 0.25) (layer "B.Cu") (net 4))
 (segment (start 145.754009 104.14) (end 147.32 104.14) (width 0.25) (layer "B.Cu") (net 4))
 (segment (start 147.32 104.14) (end 147.32 93.98) (width 0.25) (layer "B.Cu") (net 4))
 (segment (start 142.24 107.654009) (end 145.754009 104.14) (width 0.25) (layer "B.Cu") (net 4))
 (segment (start 147.345 93.98) (end 151.14 90.185) (width 0.25) (layer "B.Cu") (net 4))
 (segment (start 147.32 93.98) (end 147.345 93.98) (width 0.25) (layer "B.Cu") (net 4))
 (segment (start 157.48 93.98) (end 154.94 96.52) (width 0.25) (layer "B.Cu") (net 10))
 (segment (start 157.505 93.98) (end 157.48 93.98) (width 0.25) (layer "B.Cu") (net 10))
 (segment (start 154.94 96.52) (end 154.94 106.68) (width 0.25) (layer "B.Cu") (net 10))
 (segment (start 161.3 90.185) (end 157.505 93.98) (width 0.25) (layer "B.Cu") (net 10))
 (segment (start 154.94 106.68) (end 152.4 109.22) (width 0.25) (layer "B.Cu") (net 10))
 (segment (start 157.505 101.6) (end 161.3 97.805) (width 0.25) (layer "B.Cu") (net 11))
 (segment (start 154.94 109.22) (end 157.48 106.68) (width 0.25) (layer "B.Cu") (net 11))
 (segment (start 157.48 101.6) (end 157.505 101.6) (width 0.25) (layer "B.Cu") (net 11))
 (segment (start 157.48 106.68) (end 157.48 101.6) (width 0.25) (layer "B.Cu") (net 11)))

